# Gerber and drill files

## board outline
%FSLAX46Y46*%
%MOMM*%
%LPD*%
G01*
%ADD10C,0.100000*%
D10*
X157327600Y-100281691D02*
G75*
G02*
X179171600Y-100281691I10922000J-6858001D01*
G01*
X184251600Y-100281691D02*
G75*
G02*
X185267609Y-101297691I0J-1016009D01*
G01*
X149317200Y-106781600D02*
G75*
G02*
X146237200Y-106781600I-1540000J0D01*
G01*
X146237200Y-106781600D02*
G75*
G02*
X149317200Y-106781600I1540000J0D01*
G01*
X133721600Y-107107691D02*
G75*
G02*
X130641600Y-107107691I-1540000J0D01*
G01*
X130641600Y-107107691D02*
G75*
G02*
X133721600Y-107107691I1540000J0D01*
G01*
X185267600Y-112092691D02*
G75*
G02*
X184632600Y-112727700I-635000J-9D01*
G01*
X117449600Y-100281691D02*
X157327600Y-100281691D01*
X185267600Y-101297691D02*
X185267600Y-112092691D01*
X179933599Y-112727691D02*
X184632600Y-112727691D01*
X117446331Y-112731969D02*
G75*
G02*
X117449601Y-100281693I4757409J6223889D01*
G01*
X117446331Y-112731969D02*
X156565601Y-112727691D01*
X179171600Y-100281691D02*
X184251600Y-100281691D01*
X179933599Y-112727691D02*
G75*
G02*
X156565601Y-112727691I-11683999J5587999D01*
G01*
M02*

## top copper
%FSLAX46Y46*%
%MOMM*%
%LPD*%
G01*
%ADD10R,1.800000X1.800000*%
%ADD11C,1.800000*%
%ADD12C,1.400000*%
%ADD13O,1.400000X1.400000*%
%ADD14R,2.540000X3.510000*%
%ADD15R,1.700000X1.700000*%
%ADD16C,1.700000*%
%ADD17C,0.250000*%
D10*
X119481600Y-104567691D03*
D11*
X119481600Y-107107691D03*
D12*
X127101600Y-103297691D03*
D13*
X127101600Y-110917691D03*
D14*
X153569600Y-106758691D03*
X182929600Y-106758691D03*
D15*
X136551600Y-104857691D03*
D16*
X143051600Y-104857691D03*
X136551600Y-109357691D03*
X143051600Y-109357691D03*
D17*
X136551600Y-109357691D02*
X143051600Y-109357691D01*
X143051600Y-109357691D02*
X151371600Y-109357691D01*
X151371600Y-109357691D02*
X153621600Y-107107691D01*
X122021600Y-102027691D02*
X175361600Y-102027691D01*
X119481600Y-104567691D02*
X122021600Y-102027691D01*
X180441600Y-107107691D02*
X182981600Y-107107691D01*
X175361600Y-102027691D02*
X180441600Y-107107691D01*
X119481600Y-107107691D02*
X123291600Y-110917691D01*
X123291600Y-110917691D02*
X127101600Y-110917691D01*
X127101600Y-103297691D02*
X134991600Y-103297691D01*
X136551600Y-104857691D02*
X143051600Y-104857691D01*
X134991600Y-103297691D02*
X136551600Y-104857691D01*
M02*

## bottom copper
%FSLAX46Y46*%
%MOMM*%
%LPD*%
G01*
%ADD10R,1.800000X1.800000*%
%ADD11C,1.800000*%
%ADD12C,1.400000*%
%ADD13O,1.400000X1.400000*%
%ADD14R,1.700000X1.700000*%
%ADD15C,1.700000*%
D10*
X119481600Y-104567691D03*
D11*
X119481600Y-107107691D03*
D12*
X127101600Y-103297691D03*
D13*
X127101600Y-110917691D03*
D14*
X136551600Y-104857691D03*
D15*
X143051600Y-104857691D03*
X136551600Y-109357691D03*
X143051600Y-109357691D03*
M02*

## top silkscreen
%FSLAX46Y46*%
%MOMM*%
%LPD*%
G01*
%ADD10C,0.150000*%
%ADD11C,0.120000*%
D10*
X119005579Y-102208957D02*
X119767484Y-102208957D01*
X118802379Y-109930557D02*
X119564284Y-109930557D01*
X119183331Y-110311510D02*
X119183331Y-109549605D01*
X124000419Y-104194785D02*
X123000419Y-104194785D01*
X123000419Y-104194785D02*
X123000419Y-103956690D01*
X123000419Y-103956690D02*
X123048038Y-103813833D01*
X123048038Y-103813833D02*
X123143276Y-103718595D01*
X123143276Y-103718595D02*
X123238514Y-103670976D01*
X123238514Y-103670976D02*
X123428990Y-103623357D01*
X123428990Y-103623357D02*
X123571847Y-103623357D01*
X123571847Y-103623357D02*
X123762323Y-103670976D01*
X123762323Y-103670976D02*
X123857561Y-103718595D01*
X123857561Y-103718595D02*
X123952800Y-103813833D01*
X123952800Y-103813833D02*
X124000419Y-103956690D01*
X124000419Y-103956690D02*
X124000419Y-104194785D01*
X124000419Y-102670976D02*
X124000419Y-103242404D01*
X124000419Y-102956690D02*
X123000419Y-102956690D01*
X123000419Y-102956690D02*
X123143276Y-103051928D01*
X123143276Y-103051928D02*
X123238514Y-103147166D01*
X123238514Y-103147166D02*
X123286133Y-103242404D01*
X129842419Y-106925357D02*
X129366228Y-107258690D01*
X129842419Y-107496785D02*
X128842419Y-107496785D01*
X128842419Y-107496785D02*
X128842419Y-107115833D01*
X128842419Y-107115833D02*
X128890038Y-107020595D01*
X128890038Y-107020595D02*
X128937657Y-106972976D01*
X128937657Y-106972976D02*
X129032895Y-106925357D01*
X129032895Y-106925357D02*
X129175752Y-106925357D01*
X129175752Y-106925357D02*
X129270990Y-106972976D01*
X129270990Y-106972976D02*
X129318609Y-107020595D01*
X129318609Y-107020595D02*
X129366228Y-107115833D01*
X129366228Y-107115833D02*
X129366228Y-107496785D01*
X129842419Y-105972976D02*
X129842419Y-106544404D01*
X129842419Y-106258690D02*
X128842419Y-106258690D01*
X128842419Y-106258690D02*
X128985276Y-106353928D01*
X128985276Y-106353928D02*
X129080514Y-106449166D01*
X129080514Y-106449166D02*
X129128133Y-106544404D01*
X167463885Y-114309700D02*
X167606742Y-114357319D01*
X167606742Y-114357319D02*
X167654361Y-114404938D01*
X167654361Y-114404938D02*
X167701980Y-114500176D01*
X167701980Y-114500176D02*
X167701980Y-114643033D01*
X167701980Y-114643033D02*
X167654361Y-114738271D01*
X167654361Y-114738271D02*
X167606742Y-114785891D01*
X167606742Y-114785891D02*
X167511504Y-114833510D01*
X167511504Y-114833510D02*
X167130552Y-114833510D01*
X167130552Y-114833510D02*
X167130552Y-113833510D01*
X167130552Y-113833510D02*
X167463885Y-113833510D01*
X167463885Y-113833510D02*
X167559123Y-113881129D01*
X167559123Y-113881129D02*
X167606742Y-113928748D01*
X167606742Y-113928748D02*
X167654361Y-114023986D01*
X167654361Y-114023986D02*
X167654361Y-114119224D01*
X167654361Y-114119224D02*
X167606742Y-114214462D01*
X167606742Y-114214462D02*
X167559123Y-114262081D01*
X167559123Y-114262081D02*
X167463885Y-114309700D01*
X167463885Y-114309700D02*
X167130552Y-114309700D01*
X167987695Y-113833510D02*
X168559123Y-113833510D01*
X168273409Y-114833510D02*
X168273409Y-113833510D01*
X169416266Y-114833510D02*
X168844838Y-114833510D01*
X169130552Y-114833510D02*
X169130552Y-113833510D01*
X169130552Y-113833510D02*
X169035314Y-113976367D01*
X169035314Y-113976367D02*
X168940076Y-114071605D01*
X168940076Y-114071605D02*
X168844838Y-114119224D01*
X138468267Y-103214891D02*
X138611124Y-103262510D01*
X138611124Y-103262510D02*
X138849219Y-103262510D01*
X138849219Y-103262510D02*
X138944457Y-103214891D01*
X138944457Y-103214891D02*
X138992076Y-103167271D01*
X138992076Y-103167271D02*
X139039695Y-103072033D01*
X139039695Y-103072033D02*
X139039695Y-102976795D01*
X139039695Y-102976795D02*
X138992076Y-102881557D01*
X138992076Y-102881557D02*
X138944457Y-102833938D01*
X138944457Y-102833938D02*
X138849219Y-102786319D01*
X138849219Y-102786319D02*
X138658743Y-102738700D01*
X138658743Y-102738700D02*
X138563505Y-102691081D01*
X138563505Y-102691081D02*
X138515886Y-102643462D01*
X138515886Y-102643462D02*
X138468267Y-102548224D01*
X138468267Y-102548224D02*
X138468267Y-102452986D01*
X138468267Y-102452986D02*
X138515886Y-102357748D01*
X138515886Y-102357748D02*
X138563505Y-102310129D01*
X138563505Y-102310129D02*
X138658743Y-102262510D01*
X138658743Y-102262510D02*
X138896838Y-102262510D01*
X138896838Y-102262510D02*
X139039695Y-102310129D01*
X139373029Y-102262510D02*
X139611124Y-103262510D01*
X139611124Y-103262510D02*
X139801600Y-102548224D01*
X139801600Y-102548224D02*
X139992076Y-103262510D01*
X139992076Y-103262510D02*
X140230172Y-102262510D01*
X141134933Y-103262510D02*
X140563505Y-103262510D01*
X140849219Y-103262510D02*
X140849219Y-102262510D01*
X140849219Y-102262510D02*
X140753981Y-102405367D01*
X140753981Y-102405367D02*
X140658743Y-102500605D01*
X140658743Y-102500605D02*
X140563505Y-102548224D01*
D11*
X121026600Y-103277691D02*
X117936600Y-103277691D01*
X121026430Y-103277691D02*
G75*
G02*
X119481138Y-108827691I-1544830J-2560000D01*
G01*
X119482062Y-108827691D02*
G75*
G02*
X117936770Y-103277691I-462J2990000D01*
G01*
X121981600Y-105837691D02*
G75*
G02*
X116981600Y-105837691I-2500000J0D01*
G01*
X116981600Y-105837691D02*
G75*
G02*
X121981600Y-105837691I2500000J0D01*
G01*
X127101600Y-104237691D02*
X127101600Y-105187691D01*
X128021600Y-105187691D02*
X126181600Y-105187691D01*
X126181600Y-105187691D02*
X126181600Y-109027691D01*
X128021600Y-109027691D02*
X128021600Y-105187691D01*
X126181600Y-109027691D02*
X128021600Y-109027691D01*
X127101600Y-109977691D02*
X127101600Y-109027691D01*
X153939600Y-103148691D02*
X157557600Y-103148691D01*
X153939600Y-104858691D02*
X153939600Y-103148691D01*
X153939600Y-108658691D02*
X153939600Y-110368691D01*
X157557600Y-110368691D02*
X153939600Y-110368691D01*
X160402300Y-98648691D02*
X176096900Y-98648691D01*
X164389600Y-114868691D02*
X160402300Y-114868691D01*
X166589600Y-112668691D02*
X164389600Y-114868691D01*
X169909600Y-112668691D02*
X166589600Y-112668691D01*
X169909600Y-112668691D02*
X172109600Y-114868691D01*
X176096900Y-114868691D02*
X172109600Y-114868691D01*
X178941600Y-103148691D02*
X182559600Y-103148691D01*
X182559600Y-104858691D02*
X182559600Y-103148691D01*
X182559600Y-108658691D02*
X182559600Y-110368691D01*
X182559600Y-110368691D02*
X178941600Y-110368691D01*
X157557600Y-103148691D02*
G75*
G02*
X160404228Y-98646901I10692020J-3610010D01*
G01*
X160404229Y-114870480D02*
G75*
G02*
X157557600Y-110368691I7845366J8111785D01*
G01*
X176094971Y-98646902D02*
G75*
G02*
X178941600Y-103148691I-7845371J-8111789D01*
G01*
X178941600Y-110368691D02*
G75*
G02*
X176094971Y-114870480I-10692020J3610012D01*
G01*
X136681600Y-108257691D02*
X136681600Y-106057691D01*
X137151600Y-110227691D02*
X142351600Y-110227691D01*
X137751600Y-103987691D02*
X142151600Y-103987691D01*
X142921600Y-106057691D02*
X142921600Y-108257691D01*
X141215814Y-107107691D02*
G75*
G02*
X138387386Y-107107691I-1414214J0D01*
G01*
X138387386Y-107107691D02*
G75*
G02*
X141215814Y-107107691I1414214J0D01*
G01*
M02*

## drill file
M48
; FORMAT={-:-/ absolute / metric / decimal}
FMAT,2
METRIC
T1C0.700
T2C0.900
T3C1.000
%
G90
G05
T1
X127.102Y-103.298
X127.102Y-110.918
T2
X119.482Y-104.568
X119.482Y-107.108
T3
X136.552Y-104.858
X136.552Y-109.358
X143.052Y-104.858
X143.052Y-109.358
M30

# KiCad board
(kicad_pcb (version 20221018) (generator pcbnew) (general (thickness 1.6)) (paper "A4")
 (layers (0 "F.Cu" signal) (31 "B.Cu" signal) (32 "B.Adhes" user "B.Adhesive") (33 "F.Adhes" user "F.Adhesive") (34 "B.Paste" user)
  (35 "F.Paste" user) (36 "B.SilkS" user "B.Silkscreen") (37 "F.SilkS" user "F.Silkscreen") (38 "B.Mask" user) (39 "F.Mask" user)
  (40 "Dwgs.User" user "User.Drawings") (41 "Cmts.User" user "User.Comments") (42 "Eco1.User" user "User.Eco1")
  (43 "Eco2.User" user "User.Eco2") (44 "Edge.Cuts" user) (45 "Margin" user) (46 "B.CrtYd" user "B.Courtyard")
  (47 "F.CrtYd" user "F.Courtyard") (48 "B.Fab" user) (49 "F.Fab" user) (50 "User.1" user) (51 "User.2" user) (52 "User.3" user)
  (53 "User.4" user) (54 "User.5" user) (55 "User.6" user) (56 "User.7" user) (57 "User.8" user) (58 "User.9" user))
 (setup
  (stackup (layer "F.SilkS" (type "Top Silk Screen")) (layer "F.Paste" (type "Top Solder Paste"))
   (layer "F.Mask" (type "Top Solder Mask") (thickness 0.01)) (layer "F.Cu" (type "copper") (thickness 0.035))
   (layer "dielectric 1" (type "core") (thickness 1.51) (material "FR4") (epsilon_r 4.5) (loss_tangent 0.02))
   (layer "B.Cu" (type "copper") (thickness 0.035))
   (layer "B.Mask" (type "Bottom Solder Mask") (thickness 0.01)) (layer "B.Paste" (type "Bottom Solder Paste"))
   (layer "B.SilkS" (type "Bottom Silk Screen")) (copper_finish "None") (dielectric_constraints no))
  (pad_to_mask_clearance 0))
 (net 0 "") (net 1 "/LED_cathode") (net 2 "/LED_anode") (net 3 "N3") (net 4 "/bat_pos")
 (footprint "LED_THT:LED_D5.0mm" (layer "F.Cu") (at 119.4816 104.567691 -90)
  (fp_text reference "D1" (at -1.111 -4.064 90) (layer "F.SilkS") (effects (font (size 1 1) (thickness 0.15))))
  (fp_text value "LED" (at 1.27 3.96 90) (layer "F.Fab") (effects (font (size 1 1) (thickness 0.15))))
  (fp_line (start -1.29 -1.545) (end -1.29 1.545) (stroke (width 0.12) (type solid)) (layer "F.SilkS"))
  (fp_arc (start -1.29 -1.54483) (mid 2.072002 -2.880433) (end 4.26 0.000462) (stroke (width 0.12) (type solid)) (layer "F.SilkS"))
  (fp_arc (start 4.26 -0.000462) (mid 2.072002 2.880433) (end -1.29 1.54483) (stroke (width 0.12) (type solid)) (layer "F.SilkS"))
  (fp_circle (center 1.27 0) (end 3.77 0) (stroke (width 0.12) (type solid)) (fill none) (layer "F.SilkS"))
  (pad "1" thru_hole rect (at 0 0 270) (size 1.8 1.8) (drill 0.9) (layers "*.Cu" "*.Mask") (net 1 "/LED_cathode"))
  (pad "2" thru_hole circle (at 2.54 0 270) (size 1.8 1.8) (drill 0.9) (layers "*.Cu" "*.Mask") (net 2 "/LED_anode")))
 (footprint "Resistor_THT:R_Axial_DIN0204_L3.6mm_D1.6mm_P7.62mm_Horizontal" (layer "F.Cu") (at 127.1016 103.297691 -90)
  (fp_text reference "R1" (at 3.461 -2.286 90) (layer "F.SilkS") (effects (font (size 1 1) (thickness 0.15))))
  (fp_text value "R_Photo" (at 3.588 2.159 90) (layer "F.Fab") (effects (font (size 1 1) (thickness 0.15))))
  (fp_line (start 0.94 0) (end 1.89 0) (stroke (width 0.12) (type solid)) (layer "F.SilkS"))
  (fp_line (start 1.89 -0.92) (end 1.89 0.92) (stroke (width 0.12) (type solid)) (layer "F.SilkS"))
  (fp_line (start 1.89 0.92) (end 5.73 0.92) (stroke (width 0.12) (type solid)) (layer "F.SilkS"))
  (fp_line (start 5.73 -0.92) (end 1.89 -0.92) (stroke (width 0.12) (type solid)) (layer "F.SilkS"))
  (fp_line (start 5.73 0.92) (end 5.73 -0.92) (stroke (width 0.12) (type solid)) (layer "F.SilkS"))
  (fp_line (start 6.68 0) (end 5.73 0) (stroke (width 0.12) (type solid)) (layer "F.SilkS"))
  (pad "1" thru_hole circle (at 0 0 270) (size 1.4 1.4) (drill 0.7) (layers "*.Cu" "*.Mask") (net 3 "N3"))
  (pad "2" thru_hole oval (at 7.62 0 270) (size 1.4 1.4) (drill 0.7) (layers "*.Cu" "*.Mask") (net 2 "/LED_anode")))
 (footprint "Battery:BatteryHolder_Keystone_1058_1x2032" (layer "F.Cu") (at 168.2496 106.758691)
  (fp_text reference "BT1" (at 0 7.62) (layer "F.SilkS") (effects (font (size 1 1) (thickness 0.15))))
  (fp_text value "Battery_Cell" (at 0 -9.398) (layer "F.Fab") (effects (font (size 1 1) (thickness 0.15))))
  (fp_line (start -14.31 -3.61) (end -10.692 -3.61) (stroke (width 0.12) (type solid)) (layer "F.SilkS"))
  (fp_line (start -14.31 -1.9) (end -14.31 -3.61) (stroke (width 0.12) (type solid)) (layer "F.SilkS"))
  (fp_line (start -14.31 1.9) (end -14.31 3.61) (stroke (width 0.12) (type solid)) (layer "F.SilkS"))
  (fp_line (start -10.692 3.61) (end -14.31 3.61) (stroke (width 0.12) (type solid)) (layer "F.SilkS"))
  (fp_line (start -7.8473 -8.11) (end 7.8473 -8.11) (stroke (width 0.12) (type solid)) (layer "F.SilkS"))
  (fp_line (start -3.86 8.11) (end -7.8473 8.11) (stroke (width 0.12) (type solid)) (layer "F.SilkS"))
  (fp_line (start -1.66 5.91) (end -3.86 8.11) (stroke (width 0.12) (type solid)) (layer "F.SilkS"))
  (fp_line (start 1.66 5.91) (end -1.66 5.91) (stroke (width 0.12) (type solid)) (layer "F.SilkS"))
  (fp_line (start 1.66 5.91) (end 3.86 8.11) (stroke (width 0.12) (type solid)) (layer "F.SilkS"))
  (fp_line (start 7.8473 8.11) (end 3.86 8.11) (stroke (width 0.12) (type solid)) (layer "F.SilkS"))
  (fp_line (start 10.692 -3.61) (end 14.31 -3.61) (stroke (width 0.12) (type solid)) (layer "F.SilkS"))
  (fp_line (start 14.31 -1.9) (end 14.31 -3.61) (stroke (width 0.12) (type solid)) (layer "F.SilkS"))
  (fp_line (start 14.31 1.9) (end 14.31 3.61) (stroke (width 0.12) (type solid)) (layer "F.SilkS"))
  (fp_line (start 14.31 3.61) (end 10.692 3.61) (stroke (width 0.12) (type solid)) (layer "F.SilkS"))
  (fp_arc (start -10.692 -3.61) (mid -9.538084 -6.031244) (end -7.845371 -8.111789) (stroke (width 0.12) (type solid)) (layer "F.SilkS"))
  (fp_arc (start -7.845371 8.111789) (mid -9.538085 6.031244) (end -10.692 3.61) (stroke (width 0.12) (type solid)) (layer "F.SilkS"))
  (fp_arc (start 7.845371 -8.111789) (mid 9.538085 -6.031244) (end 10.692 -3.61) (stroke (width 0.12) (type solid)) (layer "F.SilkS"))
  (fp_arc (start 10.692 3.61) (mid 9.538084 6.031244) (end 7.845371 8.111789) (stroke (width 0.12) (type solid)) (layer "F.SilkS"))
  (pad "1" smd rect (at -14.68 0) (size 2.54 3.51) (layers "F.Cu" "F.Paste" "F.Mask") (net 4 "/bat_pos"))
  (pad "2" smd rect (at 14.68 0) (size 2.54 3.51) (layers "F.Cu" "F.Paste" "F.Mask") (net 1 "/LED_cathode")))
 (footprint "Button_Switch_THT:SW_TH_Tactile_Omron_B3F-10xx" (layer "F.Cu") (at 136.5516 104.857691)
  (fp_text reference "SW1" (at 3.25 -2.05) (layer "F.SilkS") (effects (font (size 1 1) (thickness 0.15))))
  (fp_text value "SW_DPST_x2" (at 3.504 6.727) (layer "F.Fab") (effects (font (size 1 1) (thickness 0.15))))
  (fp_line (start 0.13 3.4) (end 0.13 1.2) (stroke (width 0.12) (type solid)) (layer "F.SilkS"))
  (fp_line (start 0.6 5.37) (end 5.8 5.37) (stroke (width 0.12) (type solid)) (layer "F.SilkS"))
  (fp_line (start 1.2 -0.87) (end 5.6 -0.87) (stroke (width 0.12) (type solid)) (layer "F.SilkS"))
  (fp_line (start 6.37 1.2) (end 6.37 3.4) (stroke (width 0.12) (type solid)) (layer "F.SilkS"))
  (fp_circle (center 3.25 2.25) (end 4.25 3.25) (stroke (width 0.12) (type solid)) (fill none) (layer "F.SilkS"))
  (pad "1" thru_hole rect (at 0 0) (size 1.7 1.7) (drill 1) (layers "*.Cu" "*.Mask") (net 3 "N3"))
  (pad "1" thru_hole circle (at 6.5 0) (size 1.7 1.7) (drill 1) (layers "*.Cu" "*.Mask") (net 3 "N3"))
  (pad "2" thru_hole circle (at 0 4.5) (size 1.7 1.7) (drill 1) (layers "*.Cu" "*.Mask") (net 4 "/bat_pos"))
  (pad "2" thru_hole circle (at 6.5 4.5) (size 1.7 1.7) (drill 1) (layers "*.Cu" "*.Mask") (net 4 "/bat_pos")))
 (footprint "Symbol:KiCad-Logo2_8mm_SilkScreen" (layer "B.Cu") (at 168.1226 105.615691 180)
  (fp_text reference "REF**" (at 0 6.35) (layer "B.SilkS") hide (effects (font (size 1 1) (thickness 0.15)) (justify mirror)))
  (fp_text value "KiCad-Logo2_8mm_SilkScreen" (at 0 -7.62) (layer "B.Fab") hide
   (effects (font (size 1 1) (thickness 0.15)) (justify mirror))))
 (gr_arc (start 157.3276 100.281691) (mid 168.2496 94.243093) (end 179.1716 100.281691) (stroke (width 0.1) (type default))
  (layer "Edge.Cuts"))
 (gr_arc (start 184.2516 100.281691) (mid 184.97002 100.579271) (end 185.2676 101.297691) (stroke (width 0.1) (type default))
  (layer "Edge.Cuts"))
 (gr_circle (center 147.7772 106.7816) (end 147.7772 108.3216) (stroke (width 0.1) (type default)) (fill none) (layer "Edge.Cuts"))
 (gr_circle (center 132.1816 107.107691) (end 132.1816 108.647691) (stroke (width 0.1) (type default)) (fill none) (layer "Edge.Cuts"))
 (gr_arc (start 185.2676 112.092691) (mid 185.081613 112.541704) (end 184.6326 112.727691) (stroke (width 0.1) (type default))
  (layer "Edge.Cuts"))
 (gr_line (start 117.4496 100.281691) (end 157.3276 100.281691) (stroke (width 0.1) (type default)) (layer "Edge.Cuts"))
 (gr_line (start 185.2676 101.297691) (end 185.2676 112.092691) (stroke (width 0.1) (type default)) (layer "Edge.Cuts"))
 (gr_line (start 179.933599 112.727691) (end 184.6326 112.727691) (stroke (width 0.1) (type default)) (layer "Edge.Cuts"))
 (gr_arc (start 117.446331 112.731969) (mid 114.369857 106.506023) (end 117.4496 100.281691) (stroke (width 0.1) (type default))
  (layer "Edge.Cuts"))
 (gr_line (start 117.446331 112.731969) (end 156.565601 112.727691) (stroke (width 0.1) (type default)) (layer "Edge.Cuts"))
 (gr_line (start 179.1716 100.281691) (end 184.2516 100.281691) (stroke (width 0.1) (type default)) (layer "Edge.Cuts"))
 (gr_arc (start 179.933599 112.727691) (mid 168.2496 120.0912) (end 156.565601 112.727691) (stroke (width 0.1) (type default))
  (layer "Edge.Cuts"))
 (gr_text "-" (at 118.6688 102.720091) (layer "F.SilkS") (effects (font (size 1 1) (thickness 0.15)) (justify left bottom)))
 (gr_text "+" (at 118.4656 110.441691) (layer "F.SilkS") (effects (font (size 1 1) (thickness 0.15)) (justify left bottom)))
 (segment (start 136.5516 109.357691) (end 143.0516 109.357691) (width 0.25) (layer "F.Cu") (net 4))
 (segment (start 143.0516 109.357691) (end 151.3716 109.357691) (width 0.25) (layer "F.Cu") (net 4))
 (segment (start 151.3716 109.357691) (end 153.6216 107.107691) (width 0.25) (layer "F.Cu") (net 4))
 (segment (start 122.0216 102.027691) (end 175.3616 102.027691) (width 0.25) (layer "F.Cu") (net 1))
 (segment (start 119.4816 104.567691) (end 122.0216 102.027691) (width 0.25) (layer "F.Cu") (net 1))
 (segment (start 180.4416 107.107691) (end 182.9816 107.107691) (width 0.25) (layer "F.Cu") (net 1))
 (segment (start 175.3616 102.027691) (end 180.4416 107.107691) (width 0.25) (layer "F.Cu") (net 1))
 (segment (start 119.4816 107.107691) (end 123.2916 110.917691) (width 0.25) (layer "F.Cu") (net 2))
 (segment (start 123.2916 110.917691) (end 127.1016 110.917691) (width 0.25) (layer "F.Cu") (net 2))
 (segment (start 127.1016 103.297691) (end 134.9916 103.297691) (width 0.25) (layer "F.Cu") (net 3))
 (segment (start 136.5516 104.857691) (end 143.0516 104.857691) (width 0.25) (layer "F.Cu") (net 3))
 (segment (start 134.9916 103.297691) (end 136.5516 104.857691) (width 0.25) (layer "F.Cu") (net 3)))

